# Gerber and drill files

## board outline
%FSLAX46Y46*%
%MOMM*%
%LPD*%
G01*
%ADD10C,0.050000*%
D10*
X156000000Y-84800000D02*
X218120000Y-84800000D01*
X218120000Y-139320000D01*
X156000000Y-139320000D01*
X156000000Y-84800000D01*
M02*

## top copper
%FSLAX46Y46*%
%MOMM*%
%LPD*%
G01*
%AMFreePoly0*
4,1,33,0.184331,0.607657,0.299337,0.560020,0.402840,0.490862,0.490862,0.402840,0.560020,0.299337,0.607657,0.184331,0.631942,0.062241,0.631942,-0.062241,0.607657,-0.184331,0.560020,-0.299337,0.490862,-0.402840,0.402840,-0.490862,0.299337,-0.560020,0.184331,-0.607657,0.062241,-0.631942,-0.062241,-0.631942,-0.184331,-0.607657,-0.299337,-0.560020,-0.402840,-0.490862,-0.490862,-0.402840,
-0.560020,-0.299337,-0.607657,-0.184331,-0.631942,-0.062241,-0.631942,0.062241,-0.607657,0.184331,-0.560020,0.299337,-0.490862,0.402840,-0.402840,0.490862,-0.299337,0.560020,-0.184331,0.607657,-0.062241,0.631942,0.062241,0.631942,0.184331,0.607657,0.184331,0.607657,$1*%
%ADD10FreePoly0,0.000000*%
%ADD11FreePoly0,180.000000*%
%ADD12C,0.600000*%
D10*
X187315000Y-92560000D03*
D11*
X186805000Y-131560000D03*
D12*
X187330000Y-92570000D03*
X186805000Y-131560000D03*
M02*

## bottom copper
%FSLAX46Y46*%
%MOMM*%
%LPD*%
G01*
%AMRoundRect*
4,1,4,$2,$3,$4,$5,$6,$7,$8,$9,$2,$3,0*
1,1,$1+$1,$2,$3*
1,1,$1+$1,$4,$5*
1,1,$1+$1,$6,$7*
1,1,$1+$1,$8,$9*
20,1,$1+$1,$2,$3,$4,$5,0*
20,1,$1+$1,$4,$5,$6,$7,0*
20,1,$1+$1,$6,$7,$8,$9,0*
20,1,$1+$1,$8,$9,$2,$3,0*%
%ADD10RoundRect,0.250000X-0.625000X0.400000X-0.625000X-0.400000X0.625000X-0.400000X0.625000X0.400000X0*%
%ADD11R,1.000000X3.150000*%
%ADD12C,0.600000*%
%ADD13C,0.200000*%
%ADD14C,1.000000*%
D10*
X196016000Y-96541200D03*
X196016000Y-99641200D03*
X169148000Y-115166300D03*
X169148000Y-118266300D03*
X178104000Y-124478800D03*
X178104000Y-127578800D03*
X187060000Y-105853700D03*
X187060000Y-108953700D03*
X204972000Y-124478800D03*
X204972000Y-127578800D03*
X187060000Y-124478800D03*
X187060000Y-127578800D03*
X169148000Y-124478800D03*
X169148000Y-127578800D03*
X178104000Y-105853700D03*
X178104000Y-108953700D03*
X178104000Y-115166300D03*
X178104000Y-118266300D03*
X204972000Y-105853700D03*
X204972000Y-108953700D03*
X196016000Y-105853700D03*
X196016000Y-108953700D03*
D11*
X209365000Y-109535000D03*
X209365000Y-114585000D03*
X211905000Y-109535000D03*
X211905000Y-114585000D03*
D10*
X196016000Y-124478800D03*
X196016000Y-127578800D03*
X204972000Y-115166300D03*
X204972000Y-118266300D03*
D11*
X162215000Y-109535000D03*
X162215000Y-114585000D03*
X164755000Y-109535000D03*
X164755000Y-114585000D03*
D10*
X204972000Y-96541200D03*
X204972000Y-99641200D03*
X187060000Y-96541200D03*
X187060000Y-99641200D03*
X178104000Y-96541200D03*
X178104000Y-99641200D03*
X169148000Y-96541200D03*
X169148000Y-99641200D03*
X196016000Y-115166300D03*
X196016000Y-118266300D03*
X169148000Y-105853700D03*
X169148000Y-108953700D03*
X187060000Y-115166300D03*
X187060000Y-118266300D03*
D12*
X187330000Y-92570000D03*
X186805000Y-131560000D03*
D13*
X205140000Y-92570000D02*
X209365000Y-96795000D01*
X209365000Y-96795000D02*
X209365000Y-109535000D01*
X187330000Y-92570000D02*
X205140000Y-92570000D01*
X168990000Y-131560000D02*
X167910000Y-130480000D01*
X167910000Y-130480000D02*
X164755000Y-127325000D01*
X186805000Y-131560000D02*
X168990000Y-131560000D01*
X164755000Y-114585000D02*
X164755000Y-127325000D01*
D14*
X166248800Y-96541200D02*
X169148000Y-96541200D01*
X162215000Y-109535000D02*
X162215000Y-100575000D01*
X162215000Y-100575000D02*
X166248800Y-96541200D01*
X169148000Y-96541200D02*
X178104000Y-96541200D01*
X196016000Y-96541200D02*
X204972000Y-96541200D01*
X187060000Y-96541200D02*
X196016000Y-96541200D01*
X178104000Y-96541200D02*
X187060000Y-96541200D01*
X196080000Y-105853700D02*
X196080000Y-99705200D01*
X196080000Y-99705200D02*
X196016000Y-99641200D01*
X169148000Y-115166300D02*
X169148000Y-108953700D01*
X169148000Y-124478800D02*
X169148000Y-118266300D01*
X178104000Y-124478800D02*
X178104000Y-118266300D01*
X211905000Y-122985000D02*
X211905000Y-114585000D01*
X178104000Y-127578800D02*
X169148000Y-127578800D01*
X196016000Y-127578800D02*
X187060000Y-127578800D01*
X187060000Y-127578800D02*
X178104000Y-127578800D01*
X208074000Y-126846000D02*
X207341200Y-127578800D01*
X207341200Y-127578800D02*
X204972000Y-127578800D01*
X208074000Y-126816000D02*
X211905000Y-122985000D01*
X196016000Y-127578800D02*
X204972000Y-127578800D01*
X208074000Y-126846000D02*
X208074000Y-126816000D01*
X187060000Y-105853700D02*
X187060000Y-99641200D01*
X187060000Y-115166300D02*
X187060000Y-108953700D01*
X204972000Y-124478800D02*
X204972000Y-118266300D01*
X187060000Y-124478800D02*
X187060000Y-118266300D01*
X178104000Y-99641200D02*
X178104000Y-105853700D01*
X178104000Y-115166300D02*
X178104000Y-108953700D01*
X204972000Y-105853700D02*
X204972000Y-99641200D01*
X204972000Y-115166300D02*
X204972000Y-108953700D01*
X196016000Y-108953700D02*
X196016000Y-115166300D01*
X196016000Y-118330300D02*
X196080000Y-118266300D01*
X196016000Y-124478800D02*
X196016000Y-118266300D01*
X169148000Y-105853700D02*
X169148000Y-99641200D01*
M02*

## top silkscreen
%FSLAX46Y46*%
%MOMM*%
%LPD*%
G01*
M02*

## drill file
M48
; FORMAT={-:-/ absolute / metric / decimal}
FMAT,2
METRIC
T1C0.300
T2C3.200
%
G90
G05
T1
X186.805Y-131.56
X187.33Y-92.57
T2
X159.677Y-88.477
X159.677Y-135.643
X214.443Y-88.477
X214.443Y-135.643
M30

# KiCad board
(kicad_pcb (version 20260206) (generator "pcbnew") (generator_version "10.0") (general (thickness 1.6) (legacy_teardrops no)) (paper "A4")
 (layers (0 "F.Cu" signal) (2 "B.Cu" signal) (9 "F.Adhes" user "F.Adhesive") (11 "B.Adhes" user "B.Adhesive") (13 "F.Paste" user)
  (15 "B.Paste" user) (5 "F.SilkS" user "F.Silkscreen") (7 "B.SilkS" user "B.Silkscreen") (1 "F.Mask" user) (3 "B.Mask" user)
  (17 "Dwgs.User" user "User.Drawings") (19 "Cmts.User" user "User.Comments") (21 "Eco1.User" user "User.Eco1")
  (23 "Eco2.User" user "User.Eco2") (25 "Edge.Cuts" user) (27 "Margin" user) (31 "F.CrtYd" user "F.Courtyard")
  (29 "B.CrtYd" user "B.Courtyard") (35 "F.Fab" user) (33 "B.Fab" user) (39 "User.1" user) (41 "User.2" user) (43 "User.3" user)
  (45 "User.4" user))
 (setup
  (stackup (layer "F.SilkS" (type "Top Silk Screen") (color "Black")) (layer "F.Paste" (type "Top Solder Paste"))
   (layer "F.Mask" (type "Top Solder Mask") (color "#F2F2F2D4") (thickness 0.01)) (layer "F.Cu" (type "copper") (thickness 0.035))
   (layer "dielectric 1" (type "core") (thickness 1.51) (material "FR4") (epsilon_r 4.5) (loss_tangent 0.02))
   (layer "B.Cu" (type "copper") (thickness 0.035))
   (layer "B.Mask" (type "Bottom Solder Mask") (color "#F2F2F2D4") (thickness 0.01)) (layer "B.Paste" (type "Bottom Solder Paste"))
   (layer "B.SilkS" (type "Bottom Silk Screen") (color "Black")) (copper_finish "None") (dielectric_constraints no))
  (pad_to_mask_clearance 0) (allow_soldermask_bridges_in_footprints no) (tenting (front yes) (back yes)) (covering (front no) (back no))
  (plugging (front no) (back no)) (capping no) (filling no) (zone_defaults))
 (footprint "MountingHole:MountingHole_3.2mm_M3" (layer "F.Cu") (at 159.676955 88.476955)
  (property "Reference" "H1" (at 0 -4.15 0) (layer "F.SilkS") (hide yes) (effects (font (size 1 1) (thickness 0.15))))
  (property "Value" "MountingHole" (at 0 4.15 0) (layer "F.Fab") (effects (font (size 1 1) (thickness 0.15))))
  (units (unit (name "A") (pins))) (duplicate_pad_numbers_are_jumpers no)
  (pad "" np_thru_hole circle (at 0 0) (size 3.2 3.2) (drill 3.2) (layers "*.Cu" "*.Mask")))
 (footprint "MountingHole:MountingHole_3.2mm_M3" (layer "F.Cu") (at 214.443045 88.476955)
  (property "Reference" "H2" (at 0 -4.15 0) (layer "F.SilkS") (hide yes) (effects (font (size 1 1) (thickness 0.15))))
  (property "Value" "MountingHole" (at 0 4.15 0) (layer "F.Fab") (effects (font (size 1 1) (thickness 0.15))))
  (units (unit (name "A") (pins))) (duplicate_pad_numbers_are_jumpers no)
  (pad "" np_thru_hole circle (at 0 0) (size 3.2 3.2) (drill 3.2) (layers "*.Cu" "*.Mask")))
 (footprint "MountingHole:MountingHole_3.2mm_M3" (layer "F.Cu") (at 214.443045 135.643045)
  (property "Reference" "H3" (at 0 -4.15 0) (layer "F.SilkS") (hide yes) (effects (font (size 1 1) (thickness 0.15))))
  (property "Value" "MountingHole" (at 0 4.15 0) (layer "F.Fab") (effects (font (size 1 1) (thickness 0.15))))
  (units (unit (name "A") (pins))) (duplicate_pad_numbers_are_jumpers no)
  (pad "" np_thru_hole circle (at 0 0) (size 3.2 3.2) (drill 3.2) (layers "*.Cu" "*.Mask")))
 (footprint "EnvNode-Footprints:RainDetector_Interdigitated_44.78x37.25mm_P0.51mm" (layer "F.Cu") (at 187.315 112.06)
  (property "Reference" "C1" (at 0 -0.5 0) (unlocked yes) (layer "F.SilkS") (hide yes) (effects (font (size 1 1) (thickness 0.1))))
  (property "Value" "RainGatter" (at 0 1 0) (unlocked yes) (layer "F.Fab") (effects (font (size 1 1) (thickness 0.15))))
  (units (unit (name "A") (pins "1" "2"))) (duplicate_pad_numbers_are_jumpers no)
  (pad "1" smd custom (at 0 -19.5) (size 1.27 1.27) (layers "F.Cu") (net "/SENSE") (options (clearance outline) (anchor circle))
   (primitives))
  (pad "2" smd custom (at -0.51 19.5 180) (size 1.27 1.27) (layers "F.Cu") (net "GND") (options (clearance outline) (anchor circle))
   (primitives)))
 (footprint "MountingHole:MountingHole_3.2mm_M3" (layer "F.Cu") (at 159.676955 135.643045)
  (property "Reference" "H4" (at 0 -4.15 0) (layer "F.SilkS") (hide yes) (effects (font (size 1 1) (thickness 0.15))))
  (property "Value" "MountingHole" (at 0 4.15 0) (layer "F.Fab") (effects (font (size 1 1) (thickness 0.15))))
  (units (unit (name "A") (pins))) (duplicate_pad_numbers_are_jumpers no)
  (pad "" np_thru_hole circle (at 0 0) (size 3.2 3.2) (drill 3.2) (layers "*.Cu" "*.Mask")))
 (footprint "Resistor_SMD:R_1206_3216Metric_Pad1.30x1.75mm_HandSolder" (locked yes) (layer "B.Cu") (at 196.016 98.0912 -90)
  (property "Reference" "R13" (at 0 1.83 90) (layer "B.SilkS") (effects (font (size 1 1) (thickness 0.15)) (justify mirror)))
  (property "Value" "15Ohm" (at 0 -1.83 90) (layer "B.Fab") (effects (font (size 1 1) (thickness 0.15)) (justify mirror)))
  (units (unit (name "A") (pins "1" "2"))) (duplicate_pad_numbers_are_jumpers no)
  (pad "1" smd roundrect (at -1.55 0 270) (size 1.3 1.75) (layers "B.Cu" "B.Mask" "B.Paste") (roundrect_rratio 0.192308) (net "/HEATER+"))
  (pad "2" smd roundrect (at 1.55 0 270) (size 1.3 1.75) (layers "B.Cu" "B.Mask" "B.Paste") (roundrect_rratio 0.192308) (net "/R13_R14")))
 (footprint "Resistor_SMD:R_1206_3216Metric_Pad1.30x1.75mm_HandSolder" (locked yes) (layer "B.Cu") (at 169.148 116.7163 -90)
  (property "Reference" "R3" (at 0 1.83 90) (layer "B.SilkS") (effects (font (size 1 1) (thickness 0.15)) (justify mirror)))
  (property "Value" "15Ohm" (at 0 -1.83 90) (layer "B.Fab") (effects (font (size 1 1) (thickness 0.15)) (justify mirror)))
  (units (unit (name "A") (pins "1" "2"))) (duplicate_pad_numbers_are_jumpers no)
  (pad "1" smd roundrect (at -1.55 0 270) (size 1.3 1.75) (layers "B.Cu" "B.Mask" "B.Paste") (roundrect_rratio 0.192308) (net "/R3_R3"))
  (pad "2" smd roundrect (at 1.55 0 270) (size 1.3 1.75) (layers "B.Cu" "B.Mask" "B.Paste") (roundrect_rratio 0.192308) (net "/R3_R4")))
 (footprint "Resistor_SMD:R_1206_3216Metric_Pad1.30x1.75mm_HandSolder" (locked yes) (layer "B.Cu") (at 178.104 126.0288 -90)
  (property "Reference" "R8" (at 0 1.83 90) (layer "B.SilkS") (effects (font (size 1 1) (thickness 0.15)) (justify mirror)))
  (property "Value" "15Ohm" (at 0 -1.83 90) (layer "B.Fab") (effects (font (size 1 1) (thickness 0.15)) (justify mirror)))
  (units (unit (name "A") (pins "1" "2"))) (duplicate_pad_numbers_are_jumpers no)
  (pad "1" smd roundrect (at -1.55 0 270) (size 1.3 1.75) (layers "B.Cu" "B.Mask" "B.Paste") (roundrect_rratio 0.192308) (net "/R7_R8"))
  (pad "2" smd roundrect (at 1.55 0 270) (size 1.3 1.75) (layers "B.Cu" "B.Mask" "B.Paste") (roundrect_rratio 0.192308) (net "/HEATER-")))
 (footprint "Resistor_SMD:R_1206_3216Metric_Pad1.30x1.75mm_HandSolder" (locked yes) (layer "B.Cu") (at 187.06 107.4037 -90)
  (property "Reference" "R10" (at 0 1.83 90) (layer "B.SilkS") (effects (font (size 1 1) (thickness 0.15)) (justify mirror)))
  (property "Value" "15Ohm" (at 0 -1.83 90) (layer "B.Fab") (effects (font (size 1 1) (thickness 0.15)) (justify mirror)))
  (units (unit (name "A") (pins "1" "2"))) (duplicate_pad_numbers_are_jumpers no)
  (pad "1" smd roundrect (at -1.55 0 270) (size 1.3 1.75) (layers "B.Cu" "B.Mask" "B.Paste") (roundrect_rratio 0.192308) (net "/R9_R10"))
  (pad "2" smd roundrect (at 1.55 0 270) (size 1.3 1.75) (layers "B.Cu" "B.Mask" "B.Paste") (roundrect_rratio 0.192308) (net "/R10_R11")))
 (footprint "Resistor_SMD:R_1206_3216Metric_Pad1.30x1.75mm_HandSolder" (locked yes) (layer "B.Cu") (at 204.972 126.0288 -90)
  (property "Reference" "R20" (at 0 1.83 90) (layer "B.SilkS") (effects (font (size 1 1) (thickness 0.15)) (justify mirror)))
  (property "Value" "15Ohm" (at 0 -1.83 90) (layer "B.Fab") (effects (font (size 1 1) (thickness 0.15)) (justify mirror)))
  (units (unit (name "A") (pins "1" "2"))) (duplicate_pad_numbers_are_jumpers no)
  (pad "1" smd roundrect (at -1.55 0 270) (size 1.3 1.75) (layers "B.Cu" "B.Mask" "B.Paste") (roundrect_rratio 0.192308) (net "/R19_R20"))
  (pad "2" smd roundrect (at 1.55 0 270) (size 1.3 1.75) (layers "B.Cu" "B.Mask" "B.Paste") (roundrect_rratio 0.192308) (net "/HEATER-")))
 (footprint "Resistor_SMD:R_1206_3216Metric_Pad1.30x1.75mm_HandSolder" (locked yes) (layer "B.Cu") (at 187.06 126.0288 -90)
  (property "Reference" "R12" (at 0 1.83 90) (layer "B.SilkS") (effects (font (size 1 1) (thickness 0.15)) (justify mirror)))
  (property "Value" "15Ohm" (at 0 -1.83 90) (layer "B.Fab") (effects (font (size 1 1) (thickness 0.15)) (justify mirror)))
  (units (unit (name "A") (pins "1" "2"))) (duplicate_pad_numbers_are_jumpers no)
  (pad "1" smd roundrect (at -1.55 0 270) (size 1.3 1.75) (layers "B.Cu" "B.Mask" "B.Paste") (roundrect_rratio 0.192308) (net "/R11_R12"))
  (pad "2" smd roundrect (at 1.55 0 270) (size 1.3 1.75) (layers "B.Cu" "B.Mask" "B.Paste") (roundrect_rratio 0.192308) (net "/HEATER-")))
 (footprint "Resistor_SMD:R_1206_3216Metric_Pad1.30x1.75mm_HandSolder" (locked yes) (layer "B.Cu") (at 169.148 126.0288 -90)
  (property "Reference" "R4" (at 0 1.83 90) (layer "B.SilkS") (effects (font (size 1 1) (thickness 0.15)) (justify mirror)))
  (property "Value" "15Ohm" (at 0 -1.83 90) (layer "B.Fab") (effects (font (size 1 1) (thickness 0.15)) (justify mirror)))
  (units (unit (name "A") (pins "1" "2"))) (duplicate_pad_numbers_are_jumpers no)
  (pad "1" smd roundrect (at -1.55 0 270) (size 1.3 1.75) (layers "B.Cu" "B.Mask" "B.Paste") (roundrect_rratio 0.192308) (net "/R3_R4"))
  (pad "2" smd roundrect (at 1.55 0 270) (size 1.3 1.75) (layers "B.Cu" "B.Mask" "B.Paste") (roundrect_rratio 0.192308) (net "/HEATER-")))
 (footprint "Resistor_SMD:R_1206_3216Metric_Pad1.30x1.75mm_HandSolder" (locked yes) (layer "B.Cu") (at 178.104 107.4037 -90)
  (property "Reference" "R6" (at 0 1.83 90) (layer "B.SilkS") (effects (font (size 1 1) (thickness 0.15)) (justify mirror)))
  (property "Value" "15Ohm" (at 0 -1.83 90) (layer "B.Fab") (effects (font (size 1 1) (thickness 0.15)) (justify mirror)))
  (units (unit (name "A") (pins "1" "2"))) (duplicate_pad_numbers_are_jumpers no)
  (pad "1" smd roundrect (at -1.55 0 270) (size 1.3 1.75) (layers "B.Cu" "B.Mask" "B.Paste") (roundrect_rratio 0.192308) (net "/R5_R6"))
  (pad "2" smd roundrect (at 1.55 0 270) (size 1.3 1.75) (layers "B.Cu" "B.Mask" "B.Paste") (roundrect_rratio 0.192308) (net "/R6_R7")))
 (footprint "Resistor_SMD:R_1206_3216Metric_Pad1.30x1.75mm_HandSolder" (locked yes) (layer "B.Cu") (at 178.104 116.7163 -90)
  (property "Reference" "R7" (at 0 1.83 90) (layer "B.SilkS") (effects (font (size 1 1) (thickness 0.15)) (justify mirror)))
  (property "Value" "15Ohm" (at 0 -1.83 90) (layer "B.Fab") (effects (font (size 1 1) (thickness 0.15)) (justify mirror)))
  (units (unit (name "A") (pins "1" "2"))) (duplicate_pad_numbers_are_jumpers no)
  (pad "1" smd roundrect (at -1.55 0 270) (size 1.3 1.75) (layers "B.Cu" "B.Mask" "B.Paste") (roundrect_rratio 0.192308) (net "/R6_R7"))
  (pad "2" smd roundrect (at 1.55 0 270) (size 1.3 1.75) (layers "B.Cu" "B.Mask" "B.Paste") (roundrect_rratio 0.192308) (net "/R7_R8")))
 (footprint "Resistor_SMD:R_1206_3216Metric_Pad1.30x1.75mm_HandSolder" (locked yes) (layer "B.Cu") (at 204.972 107.4037 -90)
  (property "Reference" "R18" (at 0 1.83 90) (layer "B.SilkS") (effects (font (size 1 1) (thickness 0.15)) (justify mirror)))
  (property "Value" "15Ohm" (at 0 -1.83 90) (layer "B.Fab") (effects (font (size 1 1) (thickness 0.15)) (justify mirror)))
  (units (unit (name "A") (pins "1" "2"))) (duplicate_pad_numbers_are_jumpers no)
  (pad "1" smd roundrect (at -1.55 0 270) (size 1.3 1.75) (layers "B.Cu" "B.Mask" "B.Paste") (roundrect_rratio 0.192308) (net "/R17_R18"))
  (pad "2" smd roundrect (at 1.55 0 270) (size 1.3 1.75) (layers "B.Cu" "B.Mask" "B.Paste") (roundrect_rratio 0.192308) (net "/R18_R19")))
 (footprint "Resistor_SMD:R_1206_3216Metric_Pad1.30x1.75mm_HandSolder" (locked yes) (layer "B.Cu") (at 196.016 107.4037 -90)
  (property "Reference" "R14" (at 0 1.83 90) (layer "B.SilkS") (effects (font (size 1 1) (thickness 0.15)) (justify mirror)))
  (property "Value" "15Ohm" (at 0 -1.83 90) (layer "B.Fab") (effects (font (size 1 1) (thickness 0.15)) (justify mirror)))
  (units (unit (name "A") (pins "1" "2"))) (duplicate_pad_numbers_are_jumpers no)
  (pad "1" smd roundrect (at -1.55 0 270) (size 1.3 1.75) (layers "B.Cu" "B.Mask" "B.Paste") (roundrect_rratio 0.192308) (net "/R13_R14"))
  (pad "2" smd roundrect (at 1.55 0 270) (size 1.3 1.75) (layers "B.Cu" "B.Mask" "B.Paste") (roundrect_rratio 0.192308) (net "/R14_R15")))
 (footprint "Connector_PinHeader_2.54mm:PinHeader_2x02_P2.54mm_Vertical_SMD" (layer "B.Cu") (at 210.635 112.06 -90)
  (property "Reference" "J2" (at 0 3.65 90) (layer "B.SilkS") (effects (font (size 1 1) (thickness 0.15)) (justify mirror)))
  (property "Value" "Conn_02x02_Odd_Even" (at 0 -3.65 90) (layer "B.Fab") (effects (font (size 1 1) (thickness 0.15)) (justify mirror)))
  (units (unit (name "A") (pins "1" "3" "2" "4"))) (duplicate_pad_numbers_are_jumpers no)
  (pad "1" smd rect (at -2.525 1.27 270) (size 3.15 1) (layers "B.Cu" "B.Mask" "B.Paste") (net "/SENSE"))
  (pad "2" smd rect (at 2.525 1.27 270) (size 3.15 1) (layers "B.Cu" "B.Mask" "B.Paste") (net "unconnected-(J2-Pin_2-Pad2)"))
  (pad "3" smd rect (at -2.525 -1.27 270) (size 3.15 1) (layers "B.Cu" "B.Mask" "B.Paste") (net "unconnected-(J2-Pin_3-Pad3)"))
  (pad "4" smd rect (at 2.525 -1.27 270) (size 3.15 1) (layers "B.Cu" "B.Mask" "B.Paste") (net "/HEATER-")))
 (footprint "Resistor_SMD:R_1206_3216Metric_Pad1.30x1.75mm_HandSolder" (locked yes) (layer "B.Cu") (at 196.016 126.0288 -90)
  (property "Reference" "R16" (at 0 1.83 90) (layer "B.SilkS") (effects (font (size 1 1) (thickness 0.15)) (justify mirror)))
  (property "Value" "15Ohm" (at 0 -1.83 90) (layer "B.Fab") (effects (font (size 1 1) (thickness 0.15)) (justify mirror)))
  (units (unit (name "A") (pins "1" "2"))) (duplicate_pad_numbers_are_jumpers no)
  (pad "1" smd roundrect (at -1.55 0 270) (size 1.3 1.75) (layers "B.Cu" "B.Mask" "B.Paste") (roundrect_rratio 0.192308) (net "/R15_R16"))
  (pad "2" smd roundrect (at 1.55 0 270) (size 1.3 1.75) (layers "B.Cu" "B.Mask" "B.Paste") (roundrect_rratio 0.192308) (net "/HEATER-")))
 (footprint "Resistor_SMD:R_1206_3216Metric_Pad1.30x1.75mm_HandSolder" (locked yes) (layer "B.Cu") (at 204.972 116.7163 -90)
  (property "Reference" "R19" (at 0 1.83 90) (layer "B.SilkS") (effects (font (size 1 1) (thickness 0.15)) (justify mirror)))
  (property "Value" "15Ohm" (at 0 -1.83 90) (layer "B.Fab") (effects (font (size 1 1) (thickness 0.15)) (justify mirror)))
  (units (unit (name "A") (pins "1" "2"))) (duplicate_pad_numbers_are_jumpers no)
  (pad "1" smd roundrect (at -1.55 0 270) (size 1.3 1.75) (layers "B.Cu" "B.Mask" "B.Paste") (roundrect_rratio 0.192308) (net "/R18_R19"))
  (pad "2" smd roundrect (at 1.55 0 270) (size 1.3 1.75) (layers "B.Cu" "B.Mask" "B.Paste") (roundrect_rratio 0.192308) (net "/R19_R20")))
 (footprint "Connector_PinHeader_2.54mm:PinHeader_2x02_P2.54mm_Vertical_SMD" (layer "B.Cu") (at 163.485 112.06 -90)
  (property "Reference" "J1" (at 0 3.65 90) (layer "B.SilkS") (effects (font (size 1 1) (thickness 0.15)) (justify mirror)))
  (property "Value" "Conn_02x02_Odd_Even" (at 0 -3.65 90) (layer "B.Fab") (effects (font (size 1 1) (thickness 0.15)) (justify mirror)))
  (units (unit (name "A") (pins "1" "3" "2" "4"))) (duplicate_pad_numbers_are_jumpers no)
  (pad "1" smd rect (at -2.525 1.27 270) (size 3.15 1) (layers "B.Cu" "B.Mask" "B.Paste") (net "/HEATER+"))
  (pad "2" smd rect (at 2.525 1.27 270) (size 3.15 1) (layers "B.Cu" "B.Mask" "B.Paste") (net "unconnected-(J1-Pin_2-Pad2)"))
  (pad "3" smd rect (at -2.525 -1.27 270) (size 3.15 1) (layers "B.Cu" "B.Mask" "B.Paste") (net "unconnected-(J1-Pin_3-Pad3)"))
  (pad "4" smd rect (at 2.525 -1.27 270) (size 3.15 1) (layers "B.Cu" "B.Mask" "B.Paste") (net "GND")))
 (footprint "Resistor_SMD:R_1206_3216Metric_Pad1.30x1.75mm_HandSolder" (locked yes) (layer "B.Cu") (at 204.972 98.0912 -90)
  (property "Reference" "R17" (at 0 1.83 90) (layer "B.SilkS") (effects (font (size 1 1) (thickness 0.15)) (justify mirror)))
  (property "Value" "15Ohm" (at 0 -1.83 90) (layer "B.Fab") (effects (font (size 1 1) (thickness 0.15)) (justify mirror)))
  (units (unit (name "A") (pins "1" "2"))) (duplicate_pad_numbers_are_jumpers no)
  (pad "1" smd roundrect (at -1.55 0 270) (size 1.3 1.75) (layers "B.Cu" "B.Mask" "B.Paste") (roundrect_rratio 0.192308) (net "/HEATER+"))
  (pad "2" smd roundrect (at 1.55 0 270) (size 1.3 1.75) (layers "B.Cu" "B.Mask" "B.Paste") (roundrect_rratio 0.192308) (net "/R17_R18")))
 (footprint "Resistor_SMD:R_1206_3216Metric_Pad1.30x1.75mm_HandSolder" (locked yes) (layer "B.Cu") (at 187.06 98.0912 -90)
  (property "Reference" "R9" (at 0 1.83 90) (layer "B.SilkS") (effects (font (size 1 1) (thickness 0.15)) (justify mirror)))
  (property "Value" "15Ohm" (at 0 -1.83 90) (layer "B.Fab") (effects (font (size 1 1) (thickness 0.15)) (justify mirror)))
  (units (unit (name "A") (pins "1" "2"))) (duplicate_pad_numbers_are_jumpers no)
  (pad "1" smd roundrect (at -1.55 0 270) (size 1.3 1.75) (layers "B.Cu" "B.Mask" "B.Paste") (roundrect_rratio 0.192308) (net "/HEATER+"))
  (pad "2" smd roundrect (at 1.55 0 270) (size 1.3 1.75) (layers "B.Cu" "B.Mask" "B.Paste") (roundrect_rratio 0.192308) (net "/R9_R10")))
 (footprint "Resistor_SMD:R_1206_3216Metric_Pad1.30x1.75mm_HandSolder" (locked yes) (layer "B.Cu") (at 178.104 98.0912 -90)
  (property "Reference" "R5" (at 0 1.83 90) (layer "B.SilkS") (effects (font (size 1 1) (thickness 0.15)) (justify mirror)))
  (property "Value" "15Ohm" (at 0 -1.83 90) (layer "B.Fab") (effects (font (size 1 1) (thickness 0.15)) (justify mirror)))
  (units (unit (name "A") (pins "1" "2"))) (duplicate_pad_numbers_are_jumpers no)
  (pad "1" smd roundrect (at -1.55 0 270) (size 1.3 1.75) (layers "B.Cu" "B.Mask" "B.Paste") (roundrect_rratio 0.192308) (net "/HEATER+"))
  (pad "2" smd roundrect (at 1.55 0 270) (size 1.3 1.75) (layers "B.Cu" "B.Mask" "B.Paste") (roundrect_rratio 0.192308) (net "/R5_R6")))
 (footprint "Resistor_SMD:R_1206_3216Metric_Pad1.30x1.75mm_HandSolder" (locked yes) (layer "B.Cu") (at 169.148 98.0912 -90)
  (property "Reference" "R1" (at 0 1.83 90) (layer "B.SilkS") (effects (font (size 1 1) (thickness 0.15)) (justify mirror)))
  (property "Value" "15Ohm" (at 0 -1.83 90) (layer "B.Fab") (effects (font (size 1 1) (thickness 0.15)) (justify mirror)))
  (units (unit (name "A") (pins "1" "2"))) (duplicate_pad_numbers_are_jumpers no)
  (pad "1" smd roundrect (at -1.55 0 270) (size 1.3 1.75) (layers "B.Cu" "B.Mask" "B.Paste") (roundrect_rratio 0.192308) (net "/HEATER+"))
  (pad "2" smd roundrect (at 1.55 0 270) (size 1.3 1.75) (layers "B.Cu" "B.Mask" "B.Paste") (roundrect_rratio 0.192308) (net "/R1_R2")))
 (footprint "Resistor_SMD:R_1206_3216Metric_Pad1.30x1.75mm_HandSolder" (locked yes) (layer "B.Cu") (at 196.016 116.7163 -90)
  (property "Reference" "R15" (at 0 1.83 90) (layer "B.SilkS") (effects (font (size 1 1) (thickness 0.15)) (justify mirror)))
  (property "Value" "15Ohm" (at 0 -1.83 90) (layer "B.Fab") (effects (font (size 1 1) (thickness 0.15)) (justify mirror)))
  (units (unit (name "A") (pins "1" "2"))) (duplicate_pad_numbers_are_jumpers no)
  (pad "1" smd roundrect (at -1.55 0 270) (size 1.3 1.75) (layers "B.Cu" "B.Mask" "B.Paste") (roundrect_rratio 0.192308) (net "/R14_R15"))
  (pad "2" smd roundrect (at 1.55 0 270) (size 1.3 1.75) (layers "B.Cu" "B.Mask" "B.Paste") (roundrect_rratio 0.192308) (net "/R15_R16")))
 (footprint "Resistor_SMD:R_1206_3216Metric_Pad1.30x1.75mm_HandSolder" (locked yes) (layer "B.Cu") (at 169.148 107.4037 -90)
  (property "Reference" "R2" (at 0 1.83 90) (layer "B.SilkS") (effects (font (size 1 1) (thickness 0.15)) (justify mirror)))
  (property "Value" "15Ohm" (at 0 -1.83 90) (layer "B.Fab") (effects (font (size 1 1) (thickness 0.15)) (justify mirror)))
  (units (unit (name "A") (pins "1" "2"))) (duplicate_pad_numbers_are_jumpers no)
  (pad "1" smd roundrect (at -1.55 0 270) (size 1.3 1.75) (layers "B.Cu" "B.Mask" "B.Paste") (roundrect_rratio 0.192308) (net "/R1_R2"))
  (pad "2" smd roundrect (at 1.55 0 270) (size 1.3 1.75) (layers "B.Cu" "B.Mask" "B.Paste") (roundrect_rratio 0.192308) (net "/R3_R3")))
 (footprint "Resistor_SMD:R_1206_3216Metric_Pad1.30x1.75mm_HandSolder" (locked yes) (layer "B.Cu") (at 187.06 116.7163 -90)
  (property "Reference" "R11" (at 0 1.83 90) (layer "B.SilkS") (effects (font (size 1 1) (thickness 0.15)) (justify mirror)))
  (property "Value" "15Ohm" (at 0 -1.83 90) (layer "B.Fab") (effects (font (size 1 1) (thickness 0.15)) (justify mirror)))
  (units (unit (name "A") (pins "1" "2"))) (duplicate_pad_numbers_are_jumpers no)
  (pad "1" smd roundrect (at -1.55 0 270) (size 1.3 1.75) (layers "B.Cu" "B.Mask" "B.Paste") (roundrect_rratio 0.192308) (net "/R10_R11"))
  (pad "2" smd roundrect (at 1.55 0 270) (size 1.3 1.75) (layers "B.Cu" "B.Mask" "B.Paste") (roundrect_rratio 0.192308) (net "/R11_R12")))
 (gr_rect (start 156 84.8) (end 218.12 139.32) (stroke (width 0.05) (type solid)) (fill no) (layer "Edge.Cuts"))
 (via (at 187.33 92.57) (size 0.6) (drill 0.3) (layers "F.Cu" "B.Cu") (tenting (front yes) (back no)) (capping no)
  (covering (front no) (back no)) (plugging (front yes) (back no)) (filling no) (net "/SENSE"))
 (segment (start 205.14 92.57) (end 209.365 96.795) (width 0.2) (layer "B.Cu") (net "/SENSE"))
 (segment (start 209.365 96.795) (end 209.365 109.535) (width 0.2) (layer "B.Cu") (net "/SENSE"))
 (segment (start 187.33 92.57) (end 205.14 92.57) (width 0.2) (layer "B.Cu") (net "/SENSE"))
 (via (at 186.805 131.56) (size 0.6) (drill 0.3) (layers "F.Cu" "B.Cu") (tenting (front yes) (back no)) (capping no)
  (covering (front no) (back no)) (plugging (front yes) (back no)) (filling no) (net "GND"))
 (segment (start 168.99 131.56) (end 167.91 130.48) (width 0.2) (layer "B.Cu") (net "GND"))
 (segment (start 167.91 130.48) (end 164.755 127.325) (width 0.2) (layer "B.Cu") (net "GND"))
 (segment (start 186.805 131.56) (end 168.99 131.56) (width 0.2) (layer "B.Cu") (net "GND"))
 (segment (start 164.755 114.585) (end 164.755 127.325) (width 0.2) (layer "B.Cu") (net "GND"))
 (segment (start 166.2488 96.5412) (end 169.148 96.5412) (width 1) (layer "B.Cu") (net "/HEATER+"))
 (segment (start 162.215 109.535) (end 162.215 100.575) (width 1) (layer "B.Cu") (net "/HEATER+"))
 (segment (start 162.215 100.575) (end 166.2488 96.5412) (width 1) (layer "B.Cu") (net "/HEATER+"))
 (segment (start 169.148 96.5412) (end 178.104 96.5412) (width 1) (layer "B.Cu") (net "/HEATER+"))
 (segment (start 196.016 96.5412) (end 204.972 96.5412) (width 1) (layer "B.Cu") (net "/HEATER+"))
 (segment (start 187.06 96.5412) (end 196.016 96.5412) (width 1) (layer "B.Cu") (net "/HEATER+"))
 (segment (start 178.104 96.5412) (end 187.06 96.5412) (width 1) (layer "B.Cu") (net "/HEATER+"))
 (segment (start 196.08 105.8537) (end 196.08 99.7052) (width 1) (layer "B.Cu") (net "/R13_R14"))
 (segment (start 196.08 99.7052) (end 196.016 99.6412) (width 1) (layer "B.Cu") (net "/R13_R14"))
 (segment (start 169.148 115.1663) (end 169.148 108.9537) (width 1) (layer "B.Cu") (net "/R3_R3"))
 (segment (start 169.148 124.4788) (end 169.148 118.2663) (width 1) (layer "B.Cu") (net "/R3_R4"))
 (segment (start 178.104 124.4788) (end 178.104 118.2663) (width 1) (layer "B.Cu") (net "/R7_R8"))
 (segment (start 211.905 122.985) (end 211.905 114.585) (width 1) (layer "B.Cu") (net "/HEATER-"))
 (segment (start 178.104 127.5788) (end 169.148 127.5788) (width 1) (layer "B.Cu") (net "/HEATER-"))
 (segment (start 196.016 127.5788) (end 187.06 127.5788) (width 1) (layer "B.Cu") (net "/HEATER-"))
 (segment (start 187.06 127.5788) (end 178.104 127.5788) (width 1) (layer "B.Cu") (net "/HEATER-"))
 (segment (start 208.074 126.846) (end 207.3412 127.5788) (width 1) (layer "B.Cu") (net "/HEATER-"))
 (segment (start 207.3412 127.5788) (end 204.972 127.5788) (width 1) (layer "B.Cu") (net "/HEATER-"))
 (segment (start 208.074 126.816) (end 211.905 122.985) (width 1) (layer "B.Cu") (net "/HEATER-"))
 (segment (start 196.016 127.5788) (end 204.972 127.5788) (width 1) (layer "B.Cu") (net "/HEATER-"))
 (segment (start 208.074 126.846) (end 208.074 126.816) (width 1) (layer "B.Cu") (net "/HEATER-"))
 (segment (start 187.06 105.8537) (end 187.06 99.6412) (width 1) (layer "B.Cu") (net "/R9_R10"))
 (segment (start 187.06 115.1663) (end 187.06 108.9537) (width 1) (layer "B.Cu") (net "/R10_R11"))
 (segment (start 204.972 124.4788) (end 204.972 118.2663) (width 1) (layer "B.Cu") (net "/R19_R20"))
 (segment (start 187.06 124.4788) (end 187.06 118.2663) (width 1) (layer "B.Cu") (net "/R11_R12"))
 (segment (start 178.104 99.6412) (end 178.104 105.8537) (width 1) (layer "B.Cu") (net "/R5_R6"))
 (segment (start 178.104 115.1663) (end 178.104 108.9537) (width 1) (layer "B.Cu") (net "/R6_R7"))
 (segment (start 204.972 105.8537) (end 204.972 99.6412) (width 1) (layer "B.Cu") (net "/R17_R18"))
 (segment (start 204.972 115.1663) (end 204.972 108.9537) (width 1) (layer "B.Cu") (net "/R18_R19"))
 (segment (start 196.016 108.9537) (end 196.016 115.1663) (width 1) (layer "B.Cu") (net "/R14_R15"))
 (segment (start 196.016 118.3303) (end 196.08 118.2663) (width 1) (layer "B.Cu") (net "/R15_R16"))
 (segment (start 196.016 124.4788) (end 196.016 118.2663) (width 1) (layer "B.Cu") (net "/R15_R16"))
 (segment (start 169.148 105.8537) (end 169.148 99.6412) (width 1) (layer "B.Cu") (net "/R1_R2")))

